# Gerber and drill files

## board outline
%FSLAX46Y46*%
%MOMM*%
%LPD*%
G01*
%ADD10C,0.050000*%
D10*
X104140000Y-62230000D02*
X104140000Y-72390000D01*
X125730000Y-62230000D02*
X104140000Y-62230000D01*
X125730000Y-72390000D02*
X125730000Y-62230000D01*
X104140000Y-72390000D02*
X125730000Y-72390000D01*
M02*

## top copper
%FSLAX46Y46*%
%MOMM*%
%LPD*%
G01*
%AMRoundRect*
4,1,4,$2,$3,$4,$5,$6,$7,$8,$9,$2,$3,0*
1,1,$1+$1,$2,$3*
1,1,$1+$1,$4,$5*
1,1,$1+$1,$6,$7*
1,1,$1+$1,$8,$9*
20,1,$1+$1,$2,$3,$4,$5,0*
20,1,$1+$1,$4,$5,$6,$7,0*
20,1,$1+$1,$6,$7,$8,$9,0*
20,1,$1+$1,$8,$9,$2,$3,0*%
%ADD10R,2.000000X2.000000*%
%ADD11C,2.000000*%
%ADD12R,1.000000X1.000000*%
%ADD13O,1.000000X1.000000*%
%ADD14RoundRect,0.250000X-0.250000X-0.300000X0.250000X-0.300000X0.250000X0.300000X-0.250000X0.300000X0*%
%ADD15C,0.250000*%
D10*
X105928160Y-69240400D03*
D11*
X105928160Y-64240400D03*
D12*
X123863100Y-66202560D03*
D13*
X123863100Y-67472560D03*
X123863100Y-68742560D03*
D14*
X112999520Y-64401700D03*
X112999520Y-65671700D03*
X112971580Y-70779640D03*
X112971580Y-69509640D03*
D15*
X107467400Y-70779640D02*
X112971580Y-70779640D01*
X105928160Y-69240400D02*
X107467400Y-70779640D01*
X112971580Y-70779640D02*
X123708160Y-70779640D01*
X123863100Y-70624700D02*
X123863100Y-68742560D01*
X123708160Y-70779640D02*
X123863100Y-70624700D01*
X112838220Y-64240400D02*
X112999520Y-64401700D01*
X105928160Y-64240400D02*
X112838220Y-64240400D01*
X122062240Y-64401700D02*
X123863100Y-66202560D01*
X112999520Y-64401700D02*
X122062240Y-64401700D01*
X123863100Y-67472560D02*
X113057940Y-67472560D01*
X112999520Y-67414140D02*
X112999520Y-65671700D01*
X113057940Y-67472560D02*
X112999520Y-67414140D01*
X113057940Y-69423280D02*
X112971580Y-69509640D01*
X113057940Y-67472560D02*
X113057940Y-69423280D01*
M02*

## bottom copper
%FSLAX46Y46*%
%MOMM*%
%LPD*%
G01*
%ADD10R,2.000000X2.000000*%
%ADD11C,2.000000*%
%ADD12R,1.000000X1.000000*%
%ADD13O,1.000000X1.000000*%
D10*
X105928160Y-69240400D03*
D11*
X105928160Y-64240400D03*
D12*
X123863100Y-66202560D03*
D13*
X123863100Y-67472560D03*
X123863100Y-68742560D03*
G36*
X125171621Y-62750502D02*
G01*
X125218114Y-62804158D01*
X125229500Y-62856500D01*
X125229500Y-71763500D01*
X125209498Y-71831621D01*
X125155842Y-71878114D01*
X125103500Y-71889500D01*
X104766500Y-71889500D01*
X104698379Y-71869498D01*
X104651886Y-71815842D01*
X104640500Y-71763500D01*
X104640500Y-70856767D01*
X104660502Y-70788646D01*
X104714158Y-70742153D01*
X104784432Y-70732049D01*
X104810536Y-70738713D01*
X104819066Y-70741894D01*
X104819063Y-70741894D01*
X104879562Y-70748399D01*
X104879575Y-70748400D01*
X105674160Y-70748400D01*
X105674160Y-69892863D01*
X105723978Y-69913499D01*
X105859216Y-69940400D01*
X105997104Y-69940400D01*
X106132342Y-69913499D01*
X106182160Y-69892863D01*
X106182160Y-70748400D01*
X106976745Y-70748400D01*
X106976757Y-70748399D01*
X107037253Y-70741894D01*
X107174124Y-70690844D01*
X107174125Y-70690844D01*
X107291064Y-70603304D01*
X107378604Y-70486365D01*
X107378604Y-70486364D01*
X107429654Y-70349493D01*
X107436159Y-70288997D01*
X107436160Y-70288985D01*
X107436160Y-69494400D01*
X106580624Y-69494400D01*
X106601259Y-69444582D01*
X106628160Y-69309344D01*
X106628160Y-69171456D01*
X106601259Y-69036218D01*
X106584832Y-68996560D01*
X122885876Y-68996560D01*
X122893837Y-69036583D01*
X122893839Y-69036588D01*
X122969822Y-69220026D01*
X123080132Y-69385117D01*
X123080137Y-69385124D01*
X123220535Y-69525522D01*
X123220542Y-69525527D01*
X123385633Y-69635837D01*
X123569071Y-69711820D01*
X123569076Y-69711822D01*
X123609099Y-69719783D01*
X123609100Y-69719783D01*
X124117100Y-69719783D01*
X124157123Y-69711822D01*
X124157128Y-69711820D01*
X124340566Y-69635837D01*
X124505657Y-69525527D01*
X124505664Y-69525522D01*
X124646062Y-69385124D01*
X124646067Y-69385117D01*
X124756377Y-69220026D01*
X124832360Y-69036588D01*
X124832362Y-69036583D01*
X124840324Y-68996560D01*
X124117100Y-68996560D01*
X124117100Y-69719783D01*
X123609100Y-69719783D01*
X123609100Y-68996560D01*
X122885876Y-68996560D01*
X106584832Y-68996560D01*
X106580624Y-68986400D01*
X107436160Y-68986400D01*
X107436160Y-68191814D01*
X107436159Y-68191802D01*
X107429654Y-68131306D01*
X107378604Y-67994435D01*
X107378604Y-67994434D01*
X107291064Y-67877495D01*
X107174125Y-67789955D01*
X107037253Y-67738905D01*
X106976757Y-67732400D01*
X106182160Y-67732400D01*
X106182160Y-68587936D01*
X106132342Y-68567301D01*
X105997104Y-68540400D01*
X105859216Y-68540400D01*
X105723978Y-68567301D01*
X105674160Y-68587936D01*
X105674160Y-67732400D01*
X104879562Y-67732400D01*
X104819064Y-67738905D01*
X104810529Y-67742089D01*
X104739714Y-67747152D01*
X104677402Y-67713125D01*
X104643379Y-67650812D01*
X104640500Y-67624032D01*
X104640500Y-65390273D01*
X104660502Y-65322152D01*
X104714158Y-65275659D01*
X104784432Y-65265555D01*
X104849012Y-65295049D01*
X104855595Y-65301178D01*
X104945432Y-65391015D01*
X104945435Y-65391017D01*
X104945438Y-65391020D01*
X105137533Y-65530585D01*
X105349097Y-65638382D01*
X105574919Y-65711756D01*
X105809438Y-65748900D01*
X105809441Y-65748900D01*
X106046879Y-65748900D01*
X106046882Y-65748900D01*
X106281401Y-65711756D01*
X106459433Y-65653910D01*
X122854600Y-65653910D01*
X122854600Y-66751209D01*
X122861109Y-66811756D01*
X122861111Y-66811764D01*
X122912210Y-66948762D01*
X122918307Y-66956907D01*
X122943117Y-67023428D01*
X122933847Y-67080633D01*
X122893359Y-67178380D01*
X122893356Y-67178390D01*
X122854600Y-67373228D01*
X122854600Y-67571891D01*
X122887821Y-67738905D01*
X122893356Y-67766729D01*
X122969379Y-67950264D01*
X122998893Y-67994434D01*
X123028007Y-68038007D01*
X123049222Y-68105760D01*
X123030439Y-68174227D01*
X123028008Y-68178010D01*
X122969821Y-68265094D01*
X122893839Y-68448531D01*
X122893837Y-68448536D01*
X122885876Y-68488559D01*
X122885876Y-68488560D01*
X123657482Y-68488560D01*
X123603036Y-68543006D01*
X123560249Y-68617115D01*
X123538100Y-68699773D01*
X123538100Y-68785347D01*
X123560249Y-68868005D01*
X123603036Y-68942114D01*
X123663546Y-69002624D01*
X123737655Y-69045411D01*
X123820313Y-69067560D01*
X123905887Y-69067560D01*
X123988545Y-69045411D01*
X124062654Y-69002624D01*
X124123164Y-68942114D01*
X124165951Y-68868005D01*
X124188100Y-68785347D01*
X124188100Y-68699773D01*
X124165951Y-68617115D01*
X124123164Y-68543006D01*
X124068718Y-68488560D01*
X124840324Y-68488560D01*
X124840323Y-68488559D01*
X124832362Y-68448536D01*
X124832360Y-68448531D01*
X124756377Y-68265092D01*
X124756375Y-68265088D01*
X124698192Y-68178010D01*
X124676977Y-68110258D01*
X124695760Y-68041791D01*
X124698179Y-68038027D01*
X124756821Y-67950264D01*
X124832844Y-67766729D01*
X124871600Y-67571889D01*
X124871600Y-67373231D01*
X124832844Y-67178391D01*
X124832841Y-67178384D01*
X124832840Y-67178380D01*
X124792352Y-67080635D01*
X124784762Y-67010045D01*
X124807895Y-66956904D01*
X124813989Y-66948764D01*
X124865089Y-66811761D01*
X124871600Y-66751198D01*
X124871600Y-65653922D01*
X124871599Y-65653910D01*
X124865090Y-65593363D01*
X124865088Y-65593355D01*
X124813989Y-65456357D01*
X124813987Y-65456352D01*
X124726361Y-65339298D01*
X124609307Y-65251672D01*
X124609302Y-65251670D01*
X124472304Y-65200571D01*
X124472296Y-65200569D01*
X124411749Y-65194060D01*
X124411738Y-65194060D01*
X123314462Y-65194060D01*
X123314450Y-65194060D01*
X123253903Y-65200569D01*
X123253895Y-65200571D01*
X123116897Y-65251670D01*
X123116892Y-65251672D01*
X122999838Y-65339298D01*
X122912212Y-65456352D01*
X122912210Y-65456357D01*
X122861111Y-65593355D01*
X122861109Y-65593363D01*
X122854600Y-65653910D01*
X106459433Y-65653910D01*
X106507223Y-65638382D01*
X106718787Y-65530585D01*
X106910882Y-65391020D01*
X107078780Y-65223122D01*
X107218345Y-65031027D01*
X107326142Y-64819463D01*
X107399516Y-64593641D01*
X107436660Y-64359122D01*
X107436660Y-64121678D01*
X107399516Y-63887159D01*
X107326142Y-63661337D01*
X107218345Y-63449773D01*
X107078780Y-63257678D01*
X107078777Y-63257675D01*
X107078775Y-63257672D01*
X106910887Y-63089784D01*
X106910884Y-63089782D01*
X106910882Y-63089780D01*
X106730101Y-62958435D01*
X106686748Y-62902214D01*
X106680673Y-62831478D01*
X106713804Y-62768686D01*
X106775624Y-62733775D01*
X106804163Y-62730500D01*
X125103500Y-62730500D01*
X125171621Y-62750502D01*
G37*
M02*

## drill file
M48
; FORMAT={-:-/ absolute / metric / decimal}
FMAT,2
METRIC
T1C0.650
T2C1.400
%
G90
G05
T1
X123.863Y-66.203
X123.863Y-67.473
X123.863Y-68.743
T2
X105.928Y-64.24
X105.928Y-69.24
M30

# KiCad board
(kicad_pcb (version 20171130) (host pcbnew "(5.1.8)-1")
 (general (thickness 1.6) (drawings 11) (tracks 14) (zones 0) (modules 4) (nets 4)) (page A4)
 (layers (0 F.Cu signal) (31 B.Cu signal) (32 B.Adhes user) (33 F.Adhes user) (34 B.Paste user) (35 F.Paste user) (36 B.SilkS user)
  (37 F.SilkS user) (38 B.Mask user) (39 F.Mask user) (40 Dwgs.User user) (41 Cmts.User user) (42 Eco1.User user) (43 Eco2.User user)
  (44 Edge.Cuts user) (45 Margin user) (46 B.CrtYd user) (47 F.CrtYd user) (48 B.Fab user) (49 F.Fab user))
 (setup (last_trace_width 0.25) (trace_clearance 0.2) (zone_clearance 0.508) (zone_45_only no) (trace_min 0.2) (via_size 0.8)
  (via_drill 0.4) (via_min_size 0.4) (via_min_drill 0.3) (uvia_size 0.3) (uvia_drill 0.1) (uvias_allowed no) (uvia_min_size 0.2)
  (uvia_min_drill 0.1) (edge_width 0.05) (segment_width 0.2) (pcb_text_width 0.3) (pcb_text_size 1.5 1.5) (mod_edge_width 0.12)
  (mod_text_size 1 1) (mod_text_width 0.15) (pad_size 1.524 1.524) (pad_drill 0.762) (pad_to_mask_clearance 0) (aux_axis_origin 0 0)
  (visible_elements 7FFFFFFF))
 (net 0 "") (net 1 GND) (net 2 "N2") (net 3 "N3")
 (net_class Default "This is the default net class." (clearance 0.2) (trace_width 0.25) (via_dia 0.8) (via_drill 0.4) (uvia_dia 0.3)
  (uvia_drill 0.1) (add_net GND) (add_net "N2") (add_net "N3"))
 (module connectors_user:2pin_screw (layer F.Cu) (at 105.92816 69.2404 90)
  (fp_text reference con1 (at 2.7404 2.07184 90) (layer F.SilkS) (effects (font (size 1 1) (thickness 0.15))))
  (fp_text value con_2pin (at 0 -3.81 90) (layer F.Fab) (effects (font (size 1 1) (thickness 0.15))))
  (pad 1 thru_hole rect (at 0 0 90) (size 2 2) (drill 1.4) (layers *.Cu *.Mask) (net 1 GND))
  (pad 2 thru_hole circle (at 5 0 90) (size 2 2) (drill 1.4) (layers *.Cu *.Mask) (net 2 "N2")))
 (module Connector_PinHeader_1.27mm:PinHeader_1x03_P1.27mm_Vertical (layer F.Cu) (at 123.8631 66.20256)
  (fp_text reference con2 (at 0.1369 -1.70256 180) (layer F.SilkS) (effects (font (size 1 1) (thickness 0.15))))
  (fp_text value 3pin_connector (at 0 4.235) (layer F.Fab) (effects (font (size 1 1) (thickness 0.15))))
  (pad 1 thru_hole rect (at 0 0) (size 1 1) (drill 0.65) (layers *.Cu *.Mask) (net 2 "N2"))
  (pad 2 thru_hole oval (at 0 1.27) (size 1 1) (drill 0.65) (layers *.Cu *.Mask) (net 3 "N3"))
  (pad 3 thru_hole oval (at 0 2.54) (size 1 1) (drill 0.65) (layers *.Cu *.Mask) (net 1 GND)))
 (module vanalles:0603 (layer F.Cu) (at 112.99952 64.4017 270)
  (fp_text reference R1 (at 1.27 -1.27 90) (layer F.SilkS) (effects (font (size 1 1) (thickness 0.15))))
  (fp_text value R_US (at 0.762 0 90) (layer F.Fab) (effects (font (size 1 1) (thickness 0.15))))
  (pad 1 smd roundrect (at 0 0) (size 1 1.1) (layers F.Cu F.Paste F.Mask) (roundrect_rratio 0.25) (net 2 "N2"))
  (pad 2 smd roundrect (at 1.27 0) (size 1 1.1) (layers F.Cu F.Paste F.Mask) (roundrect_rratio 0.25) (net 3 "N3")))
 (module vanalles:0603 (layer F.Cu) (at 112.97158 69.50964 270)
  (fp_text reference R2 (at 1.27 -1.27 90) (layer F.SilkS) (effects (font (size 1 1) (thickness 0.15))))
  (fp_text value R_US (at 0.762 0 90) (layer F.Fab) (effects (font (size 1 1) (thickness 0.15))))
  (pad 2 smd roundrect (at 1.27 0) (size 1 1.1) (layers F.Cu F.Paste F.Mask) (roundrect_rratio 0.25) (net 1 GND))
  (pad 1 smd roundrect (at 0 0) (size 1 1.1) (layers F.Cu F.Paste F.Mask) (roundrect_rratio 0.25) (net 3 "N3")))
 (gr_line (start 104.14 62.23) (end 104.14 72.39) (layer Edge.Cuts) (width 0.05))
 (gr_line (start 125.73 62.23) (end 104.14 62.23) (layer Edge.Cuts) (width 0.05))
 (gr_line (start 125.73 72.39) (end 125.73 62.23) (layer Edge.Cuts) (width 0.05))
 (gr_line (start 104.14 72.39) (end 125.73 72.39) (layer Edge.Cuts) (width 0.05))
 (segment (start 107.4674 70.77964) (end 112.97158 70.77964) (width 0.25) (layer F.Cu) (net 1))
 (segment (start 105.92816 69.2404) (end 107.4674 70.77964) (width 0.25) (layer F.Cu) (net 1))
 (segment (start 112.97158 70.77964) (end 123.70816 70.77964) (width 0.25) (layer F.Cu) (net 1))
 (segment (start 123.8631 70.6247) (end 123.8631 68.74256) (width 0.25) (layer F.Cu) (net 1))
 (segment (start 123.70816 70.77964) (end 123.8631 70.6247) (width 0.25) (layer F.Cu) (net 1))
 (segment (start 112.83822 64.2404) (end 112.99952 64.4017) (width 0.25) (layer F.Cu) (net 2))
 (segment (start 105.92816 64.2404) (end 112.83822 64.2404) (width 0.25) (layer F.Cu) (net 2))
 (segment (start 122.06224 64.4017) (end 123.8631 66.20256) (width 0.25) (layer F.Cu) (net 2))
 (segment (start 112.99952 64.4017) (end 122.06224 64.4017) (width 0.25) (layer F.Cu) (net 2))
 (segment (start 123.8631 67.47256) (end 113.05794 67.47256) (width 0.25) (layer F.Cu) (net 3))
 (segment (start 112.99952 67.41414) (end 112.99952 65.6717) (width 0.25) (layer F.Cu) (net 3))
 (segment (start 113.05794 67.47256) (end 112.99952 67.41414) (width 0.25) (layer F.Cu) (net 3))
 (segment (start 113.05794 69.42328) (end 112.97158 69.50964) (width 0.25) (layer F.Cu) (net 3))
 (segment (start 113.05794 67.47256) (end 113.05794 69.42328) (width 0.25) (layer F.Cu) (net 3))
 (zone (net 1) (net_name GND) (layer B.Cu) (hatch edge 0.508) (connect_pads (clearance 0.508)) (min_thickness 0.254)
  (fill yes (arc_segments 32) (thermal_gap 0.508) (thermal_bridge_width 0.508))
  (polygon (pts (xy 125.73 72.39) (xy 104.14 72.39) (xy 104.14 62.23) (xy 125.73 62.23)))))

